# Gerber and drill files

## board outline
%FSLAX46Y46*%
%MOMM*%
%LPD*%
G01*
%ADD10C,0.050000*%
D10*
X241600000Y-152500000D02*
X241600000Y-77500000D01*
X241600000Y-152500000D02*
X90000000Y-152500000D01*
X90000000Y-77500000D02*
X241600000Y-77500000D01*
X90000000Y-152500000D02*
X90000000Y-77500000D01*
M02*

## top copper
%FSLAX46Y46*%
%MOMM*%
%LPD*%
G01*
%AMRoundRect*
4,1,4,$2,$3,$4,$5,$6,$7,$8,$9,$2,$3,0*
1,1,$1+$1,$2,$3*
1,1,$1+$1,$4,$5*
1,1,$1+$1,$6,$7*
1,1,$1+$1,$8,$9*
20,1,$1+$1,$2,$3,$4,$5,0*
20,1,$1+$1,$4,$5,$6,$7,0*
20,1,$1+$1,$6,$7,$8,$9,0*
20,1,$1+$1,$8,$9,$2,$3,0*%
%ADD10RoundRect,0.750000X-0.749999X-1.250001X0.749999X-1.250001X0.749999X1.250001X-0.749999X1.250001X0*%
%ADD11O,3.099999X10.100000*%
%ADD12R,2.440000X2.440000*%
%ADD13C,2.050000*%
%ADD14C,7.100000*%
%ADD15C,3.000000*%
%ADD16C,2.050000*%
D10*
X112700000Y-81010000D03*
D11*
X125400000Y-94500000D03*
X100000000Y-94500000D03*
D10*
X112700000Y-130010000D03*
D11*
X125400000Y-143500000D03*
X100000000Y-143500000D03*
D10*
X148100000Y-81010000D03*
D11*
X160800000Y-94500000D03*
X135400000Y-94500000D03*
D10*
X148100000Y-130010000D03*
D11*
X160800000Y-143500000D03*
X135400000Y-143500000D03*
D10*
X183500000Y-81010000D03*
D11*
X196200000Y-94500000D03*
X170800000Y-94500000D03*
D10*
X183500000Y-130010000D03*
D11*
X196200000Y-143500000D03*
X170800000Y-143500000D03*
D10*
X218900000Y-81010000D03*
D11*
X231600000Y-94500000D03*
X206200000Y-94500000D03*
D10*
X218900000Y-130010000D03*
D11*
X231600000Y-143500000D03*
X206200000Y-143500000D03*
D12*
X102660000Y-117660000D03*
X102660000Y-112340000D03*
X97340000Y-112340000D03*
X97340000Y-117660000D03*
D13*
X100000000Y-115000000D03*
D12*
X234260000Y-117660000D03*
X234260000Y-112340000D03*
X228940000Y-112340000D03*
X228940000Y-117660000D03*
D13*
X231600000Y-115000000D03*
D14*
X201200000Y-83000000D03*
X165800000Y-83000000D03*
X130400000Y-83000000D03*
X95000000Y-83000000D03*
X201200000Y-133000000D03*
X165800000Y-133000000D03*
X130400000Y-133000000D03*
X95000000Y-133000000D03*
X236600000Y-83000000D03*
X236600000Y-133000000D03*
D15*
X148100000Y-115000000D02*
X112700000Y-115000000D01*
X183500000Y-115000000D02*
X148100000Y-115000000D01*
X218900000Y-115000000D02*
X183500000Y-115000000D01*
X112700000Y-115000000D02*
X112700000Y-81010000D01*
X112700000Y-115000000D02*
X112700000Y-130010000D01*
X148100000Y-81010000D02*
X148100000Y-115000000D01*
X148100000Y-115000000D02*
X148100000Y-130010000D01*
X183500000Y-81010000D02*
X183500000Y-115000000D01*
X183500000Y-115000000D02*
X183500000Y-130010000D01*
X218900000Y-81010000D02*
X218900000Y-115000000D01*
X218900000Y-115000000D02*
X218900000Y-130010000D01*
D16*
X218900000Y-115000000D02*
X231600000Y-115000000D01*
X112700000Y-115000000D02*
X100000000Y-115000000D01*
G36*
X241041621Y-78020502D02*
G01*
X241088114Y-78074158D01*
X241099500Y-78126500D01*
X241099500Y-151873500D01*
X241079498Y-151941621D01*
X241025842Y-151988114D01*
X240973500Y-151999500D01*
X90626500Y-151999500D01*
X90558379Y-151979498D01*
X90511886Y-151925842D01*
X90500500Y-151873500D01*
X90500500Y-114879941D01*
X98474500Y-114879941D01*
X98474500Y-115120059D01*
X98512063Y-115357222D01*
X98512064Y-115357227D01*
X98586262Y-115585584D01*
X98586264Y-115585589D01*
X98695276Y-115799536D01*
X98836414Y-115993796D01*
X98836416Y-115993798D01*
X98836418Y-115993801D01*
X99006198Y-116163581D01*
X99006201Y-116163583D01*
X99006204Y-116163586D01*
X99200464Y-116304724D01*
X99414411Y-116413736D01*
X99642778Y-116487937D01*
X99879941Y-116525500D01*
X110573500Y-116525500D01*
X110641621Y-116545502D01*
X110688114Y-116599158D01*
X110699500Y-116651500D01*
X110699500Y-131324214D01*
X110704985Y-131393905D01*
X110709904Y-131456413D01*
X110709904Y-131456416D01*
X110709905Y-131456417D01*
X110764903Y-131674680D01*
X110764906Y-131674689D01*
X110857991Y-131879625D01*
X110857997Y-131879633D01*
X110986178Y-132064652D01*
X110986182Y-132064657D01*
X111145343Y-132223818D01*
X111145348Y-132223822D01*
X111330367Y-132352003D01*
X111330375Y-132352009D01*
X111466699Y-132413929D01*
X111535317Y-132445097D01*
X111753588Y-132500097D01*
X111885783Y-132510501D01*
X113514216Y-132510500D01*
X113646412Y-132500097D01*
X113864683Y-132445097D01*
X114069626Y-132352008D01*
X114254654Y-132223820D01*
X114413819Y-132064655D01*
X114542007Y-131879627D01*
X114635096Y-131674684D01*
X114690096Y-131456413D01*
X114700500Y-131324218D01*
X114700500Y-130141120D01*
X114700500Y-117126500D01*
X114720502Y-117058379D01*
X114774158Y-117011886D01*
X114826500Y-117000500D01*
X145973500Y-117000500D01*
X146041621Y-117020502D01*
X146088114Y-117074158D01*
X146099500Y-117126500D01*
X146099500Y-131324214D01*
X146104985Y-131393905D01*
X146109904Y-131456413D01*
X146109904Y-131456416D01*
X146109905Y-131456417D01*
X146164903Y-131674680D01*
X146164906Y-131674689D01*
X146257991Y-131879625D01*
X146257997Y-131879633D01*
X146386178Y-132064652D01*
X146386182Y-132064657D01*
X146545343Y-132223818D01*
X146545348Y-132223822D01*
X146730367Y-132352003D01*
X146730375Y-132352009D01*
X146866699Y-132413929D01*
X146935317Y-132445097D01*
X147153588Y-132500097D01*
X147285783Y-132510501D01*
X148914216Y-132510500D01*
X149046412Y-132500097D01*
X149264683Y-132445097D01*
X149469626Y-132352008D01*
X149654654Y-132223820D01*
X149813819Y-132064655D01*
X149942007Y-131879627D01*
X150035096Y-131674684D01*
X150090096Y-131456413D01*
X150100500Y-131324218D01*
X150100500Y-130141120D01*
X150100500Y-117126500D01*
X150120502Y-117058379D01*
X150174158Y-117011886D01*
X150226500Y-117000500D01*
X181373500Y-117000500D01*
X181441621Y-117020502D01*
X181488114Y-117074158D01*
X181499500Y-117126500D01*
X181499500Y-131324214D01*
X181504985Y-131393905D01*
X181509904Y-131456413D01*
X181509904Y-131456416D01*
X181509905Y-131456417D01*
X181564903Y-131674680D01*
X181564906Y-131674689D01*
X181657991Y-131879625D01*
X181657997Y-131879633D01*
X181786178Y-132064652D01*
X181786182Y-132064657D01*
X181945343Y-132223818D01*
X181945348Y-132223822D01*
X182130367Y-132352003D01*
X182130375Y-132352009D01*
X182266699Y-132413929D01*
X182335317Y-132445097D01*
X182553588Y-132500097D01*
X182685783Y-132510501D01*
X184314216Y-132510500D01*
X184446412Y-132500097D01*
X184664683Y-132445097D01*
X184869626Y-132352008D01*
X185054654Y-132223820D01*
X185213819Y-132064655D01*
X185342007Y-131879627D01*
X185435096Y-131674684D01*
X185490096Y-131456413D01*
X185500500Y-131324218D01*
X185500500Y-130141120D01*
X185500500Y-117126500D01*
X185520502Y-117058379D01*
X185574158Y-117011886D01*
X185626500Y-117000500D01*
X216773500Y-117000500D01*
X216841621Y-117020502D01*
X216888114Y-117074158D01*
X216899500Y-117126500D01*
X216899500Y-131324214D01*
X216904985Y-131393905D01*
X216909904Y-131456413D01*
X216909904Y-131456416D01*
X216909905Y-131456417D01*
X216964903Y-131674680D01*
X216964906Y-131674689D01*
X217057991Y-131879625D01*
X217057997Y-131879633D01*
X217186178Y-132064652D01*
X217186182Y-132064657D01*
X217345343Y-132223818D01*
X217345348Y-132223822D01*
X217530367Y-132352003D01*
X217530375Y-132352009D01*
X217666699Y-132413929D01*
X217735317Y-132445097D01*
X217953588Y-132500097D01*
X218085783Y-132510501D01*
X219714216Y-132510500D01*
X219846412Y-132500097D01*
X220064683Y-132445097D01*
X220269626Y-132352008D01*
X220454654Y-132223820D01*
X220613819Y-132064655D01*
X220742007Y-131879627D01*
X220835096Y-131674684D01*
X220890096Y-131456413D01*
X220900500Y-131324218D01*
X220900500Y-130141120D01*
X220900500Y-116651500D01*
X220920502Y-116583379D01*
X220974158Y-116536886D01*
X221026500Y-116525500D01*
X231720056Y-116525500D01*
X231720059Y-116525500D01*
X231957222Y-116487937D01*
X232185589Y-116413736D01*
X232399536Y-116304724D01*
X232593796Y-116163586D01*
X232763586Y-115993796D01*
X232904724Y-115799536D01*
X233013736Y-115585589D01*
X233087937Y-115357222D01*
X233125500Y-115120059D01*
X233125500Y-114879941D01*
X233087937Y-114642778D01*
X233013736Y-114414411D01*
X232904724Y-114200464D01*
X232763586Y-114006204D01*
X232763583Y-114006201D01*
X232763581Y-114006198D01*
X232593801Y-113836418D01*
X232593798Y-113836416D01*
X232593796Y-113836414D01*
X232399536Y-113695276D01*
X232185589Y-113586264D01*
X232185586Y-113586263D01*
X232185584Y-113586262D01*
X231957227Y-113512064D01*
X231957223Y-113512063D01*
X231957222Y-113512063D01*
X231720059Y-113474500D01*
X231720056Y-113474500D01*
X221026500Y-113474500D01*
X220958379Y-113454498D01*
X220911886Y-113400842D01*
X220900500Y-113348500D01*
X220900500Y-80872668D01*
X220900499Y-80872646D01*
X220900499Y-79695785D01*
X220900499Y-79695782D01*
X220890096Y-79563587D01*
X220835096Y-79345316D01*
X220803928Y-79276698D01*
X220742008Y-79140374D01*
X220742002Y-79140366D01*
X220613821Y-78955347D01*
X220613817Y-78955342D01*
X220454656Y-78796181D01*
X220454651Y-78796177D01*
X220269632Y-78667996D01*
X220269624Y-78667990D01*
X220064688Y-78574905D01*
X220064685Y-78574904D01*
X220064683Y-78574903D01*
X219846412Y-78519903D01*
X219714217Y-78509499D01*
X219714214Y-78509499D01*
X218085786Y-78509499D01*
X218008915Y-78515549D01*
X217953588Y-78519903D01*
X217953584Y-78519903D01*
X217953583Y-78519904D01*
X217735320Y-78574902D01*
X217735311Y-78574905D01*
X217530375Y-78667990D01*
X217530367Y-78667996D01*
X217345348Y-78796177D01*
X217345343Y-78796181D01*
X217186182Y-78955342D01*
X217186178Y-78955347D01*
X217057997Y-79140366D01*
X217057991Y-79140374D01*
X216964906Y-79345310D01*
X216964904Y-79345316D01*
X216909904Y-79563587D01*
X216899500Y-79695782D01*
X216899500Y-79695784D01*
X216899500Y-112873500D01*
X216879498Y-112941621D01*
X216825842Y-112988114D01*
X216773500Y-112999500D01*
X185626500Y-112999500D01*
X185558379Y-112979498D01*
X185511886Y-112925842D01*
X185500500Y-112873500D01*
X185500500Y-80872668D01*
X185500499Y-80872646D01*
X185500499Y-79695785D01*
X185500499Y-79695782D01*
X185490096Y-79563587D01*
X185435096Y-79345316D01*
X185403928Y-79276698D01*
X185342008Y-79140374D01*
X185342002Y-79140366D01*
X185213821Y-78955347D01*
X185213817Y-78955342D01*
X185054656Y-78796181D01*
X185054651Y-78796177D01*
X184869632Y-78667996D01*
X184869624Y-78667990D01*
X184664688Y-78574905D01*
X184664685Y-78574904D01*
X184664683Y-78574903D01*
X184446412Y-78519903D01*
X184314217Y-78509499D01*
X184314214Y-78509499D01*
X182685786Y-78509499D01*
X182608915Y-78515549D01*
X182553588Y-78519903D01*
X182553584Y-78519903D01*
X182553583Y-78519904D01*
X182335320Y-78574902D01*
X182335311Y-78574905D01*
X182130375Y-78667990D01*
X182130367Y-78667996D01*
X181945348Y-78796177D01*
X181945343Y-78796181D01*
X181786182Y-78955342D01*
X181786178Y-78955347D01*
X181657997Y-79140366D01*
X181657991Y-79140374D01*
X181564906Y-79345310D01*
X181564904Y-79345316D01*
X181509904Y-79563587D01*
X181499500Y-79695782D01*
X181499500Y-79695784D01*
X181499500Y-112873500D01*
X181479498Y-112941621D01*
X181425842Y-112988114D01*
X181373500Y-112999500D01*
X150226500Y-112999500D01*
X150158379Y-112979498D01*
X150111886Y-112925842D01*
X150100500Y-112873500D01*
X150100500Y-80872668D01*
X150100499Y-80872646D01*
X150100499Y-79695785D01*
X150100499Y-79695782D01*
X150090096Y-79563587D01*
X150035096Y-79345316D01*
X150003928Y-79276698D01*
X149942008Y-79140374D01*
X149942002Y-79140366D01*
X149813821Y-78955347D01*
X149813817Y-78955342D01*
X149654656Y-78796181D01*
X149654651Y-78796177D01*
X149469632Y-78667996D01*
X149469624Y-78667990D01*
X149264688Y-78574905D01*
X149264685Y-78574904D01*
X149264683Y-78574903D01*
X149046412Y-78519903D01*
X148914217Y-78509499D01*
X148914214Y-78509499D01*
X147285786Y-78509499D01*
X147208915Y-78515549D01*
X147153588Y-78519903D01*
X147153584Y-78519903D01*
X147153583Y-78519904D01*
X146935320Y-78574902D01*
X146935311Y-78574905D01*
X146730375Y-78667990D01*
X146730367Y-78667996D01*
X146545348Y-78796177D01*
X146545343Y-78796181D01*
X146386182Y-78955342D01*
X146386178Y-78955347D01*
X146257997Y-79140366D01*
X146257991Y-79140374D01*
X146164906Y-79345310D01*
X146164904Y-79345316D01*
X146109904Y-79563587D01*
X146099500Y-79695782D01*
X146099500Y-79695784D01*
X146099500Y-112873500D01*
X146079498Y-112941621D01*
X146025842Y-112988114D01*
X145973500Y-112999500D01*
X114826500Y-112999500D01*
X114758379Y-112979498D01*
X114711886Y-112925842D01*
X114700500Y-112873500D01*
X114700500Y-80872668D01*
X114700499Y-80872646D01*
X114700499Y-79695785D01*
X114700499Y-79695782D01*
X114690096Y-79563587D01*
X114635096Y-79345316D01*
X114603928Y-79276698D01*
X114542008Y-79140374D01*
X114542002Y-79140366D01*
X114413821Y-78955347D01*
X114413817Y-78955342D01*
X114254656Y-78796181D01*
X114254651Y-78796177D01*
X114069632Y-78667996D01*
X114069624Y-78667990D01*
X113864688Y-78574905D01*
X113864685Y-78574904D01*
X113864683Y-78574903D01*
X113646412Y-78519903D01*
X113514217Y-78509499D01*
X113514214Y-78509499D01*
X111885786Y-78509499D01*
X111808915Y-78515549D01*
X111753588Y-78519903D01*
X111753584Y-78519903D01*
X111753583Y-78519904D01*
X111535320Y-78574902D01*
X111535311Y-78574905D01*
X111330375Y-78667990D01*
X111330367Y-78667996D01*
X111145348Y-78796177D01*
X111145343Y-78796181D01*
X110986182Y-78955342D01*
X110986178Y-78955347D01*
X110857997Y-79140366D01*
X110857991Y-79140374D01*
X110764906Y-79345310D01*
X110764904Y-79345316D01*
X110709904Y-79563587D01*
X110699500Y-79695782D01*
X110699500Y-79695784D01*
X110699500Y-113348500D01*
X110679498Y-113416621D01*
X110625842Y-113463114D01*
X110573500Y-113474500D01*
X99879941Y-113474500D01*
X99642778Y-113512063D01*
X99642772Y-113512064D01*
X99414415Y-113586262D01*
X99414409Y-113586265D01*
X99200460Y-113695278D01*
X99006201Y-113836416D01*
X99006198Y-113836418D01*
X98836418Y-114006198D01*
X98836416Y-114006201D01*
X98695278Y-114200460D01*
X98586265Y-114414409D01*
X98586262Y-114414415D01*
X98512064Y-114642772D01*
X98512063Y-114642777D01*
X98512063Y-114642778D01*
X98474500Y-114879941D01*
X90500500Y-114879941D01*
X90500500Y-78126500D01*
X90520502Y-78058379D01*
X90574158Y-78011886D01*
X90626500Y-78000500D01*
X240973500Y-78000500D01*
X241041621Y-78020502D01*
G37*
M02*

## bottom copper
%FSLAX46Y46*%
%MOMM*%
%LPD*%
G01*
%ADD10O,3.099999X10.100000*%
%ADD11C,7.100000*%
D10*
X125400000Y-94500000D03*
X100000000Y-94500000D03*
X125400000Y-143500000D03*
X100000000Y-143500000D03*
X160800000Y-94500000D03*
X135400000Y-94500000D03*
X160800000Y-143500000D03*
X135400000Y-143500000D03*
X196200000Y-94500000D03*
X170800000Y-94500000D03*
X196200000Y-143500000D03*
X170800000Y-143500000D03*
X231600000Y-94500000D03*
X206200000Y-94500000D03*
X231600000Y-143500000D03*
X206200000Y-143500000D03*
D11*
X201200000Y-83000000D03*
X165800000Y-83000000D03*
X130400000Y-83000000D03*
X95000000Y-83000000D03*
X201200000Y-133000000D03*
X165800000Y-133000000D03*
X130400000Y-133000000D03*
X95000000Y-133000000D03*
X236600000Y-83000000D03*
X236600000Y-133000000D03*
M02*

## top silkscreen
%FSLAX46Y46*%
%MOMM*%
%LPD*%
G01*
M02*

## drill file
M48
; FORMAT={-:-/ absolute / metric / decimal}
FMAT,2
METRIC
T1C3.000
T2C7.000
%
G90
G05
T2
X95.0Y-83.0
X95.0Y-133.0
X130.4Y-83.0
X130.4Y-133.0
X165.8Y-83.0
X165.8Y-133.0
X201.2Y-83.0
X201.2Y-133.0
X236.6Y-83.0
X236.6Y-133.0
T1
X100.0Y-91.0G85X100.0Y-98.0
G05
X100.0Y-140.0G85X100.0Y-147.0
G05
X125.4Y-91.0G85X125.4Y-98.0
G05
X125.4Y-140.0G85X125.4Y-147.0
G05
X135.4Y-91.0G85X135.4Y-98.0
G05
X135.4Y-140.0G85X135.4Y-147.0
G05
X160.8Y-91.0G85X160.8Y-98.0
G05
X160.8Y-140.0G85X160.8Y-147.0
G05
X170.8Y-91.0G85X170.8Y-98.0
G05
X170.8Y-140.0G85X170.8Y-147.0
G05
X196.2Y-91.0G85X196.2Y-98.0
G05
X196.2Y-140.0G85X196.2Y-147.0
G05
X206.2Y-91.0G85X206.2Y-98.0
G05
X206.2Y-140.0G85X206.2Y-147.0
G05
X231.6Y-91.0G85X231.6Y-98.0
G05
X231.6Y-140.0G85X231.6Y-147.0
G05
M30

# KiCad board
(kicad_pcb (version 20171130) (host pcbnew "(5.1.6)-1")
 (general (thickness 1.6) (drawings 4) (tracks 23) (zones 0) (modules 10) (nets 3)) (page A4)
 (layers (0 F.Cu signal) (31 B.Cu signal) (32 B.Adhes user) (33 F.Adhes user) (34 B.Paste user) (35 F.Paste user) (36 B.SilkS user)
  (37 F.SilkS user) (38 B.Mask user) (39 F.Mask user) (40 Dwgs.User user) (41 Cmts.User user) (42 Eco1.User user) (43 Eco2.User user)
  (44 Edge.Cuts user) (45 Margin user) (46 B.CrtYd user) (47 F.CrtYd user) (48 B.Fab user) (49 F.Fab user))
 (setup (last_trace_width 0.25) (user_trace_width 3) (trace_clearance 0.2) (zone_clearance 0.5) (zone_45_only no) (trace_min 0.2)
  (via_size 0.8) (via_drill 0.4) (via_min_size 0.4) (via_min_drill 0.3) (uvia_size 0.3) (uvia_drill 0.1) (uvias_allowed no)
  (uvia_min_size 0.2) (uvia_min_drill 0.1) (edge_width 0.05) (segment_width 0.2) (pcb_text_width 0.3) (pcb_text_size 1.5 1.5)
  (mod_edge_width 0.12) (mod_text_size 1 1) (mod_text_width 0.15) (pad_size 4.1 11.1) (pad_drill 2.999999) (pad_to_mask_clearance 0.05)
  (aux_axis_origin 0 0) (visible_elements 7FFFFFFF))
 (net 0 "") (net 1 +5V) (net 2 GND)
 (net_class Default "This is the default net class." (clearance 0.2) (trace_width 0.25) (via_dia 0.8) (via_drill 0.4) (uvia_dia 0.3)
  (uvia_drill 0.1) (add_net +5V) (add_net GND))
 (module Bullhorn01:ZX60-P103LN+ (layer F.Cu) (at 112.7 94.5)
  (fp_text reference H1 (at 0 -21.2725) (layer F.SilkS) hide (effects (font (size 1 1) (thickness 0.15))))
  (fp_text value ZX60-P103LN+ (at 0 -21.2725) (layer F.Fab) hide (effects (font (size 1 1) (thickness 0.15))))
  (pad 2 smd roundrect (at 0 -13.49) (size 2.999999 4.000002) (layers F.Cu F.Paste F.Mask) (roundrect_rratio 0.25) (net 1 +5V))
  (pad 1 thru_hole oval (at 12.7 0) (size 3.099999 10.1) (drill oval 2.999999 10) (layers *.Cu *.Mask) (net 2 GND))
  (pad 1 thru_hole oval (at -12.7 0) (size 3.099999 10.1) (drill oval 2.999999 10) (layers *.Cu *.Mask) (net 2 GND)))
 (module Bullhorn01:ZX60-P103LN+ (layer F.Cu) (at 112.7 143.5)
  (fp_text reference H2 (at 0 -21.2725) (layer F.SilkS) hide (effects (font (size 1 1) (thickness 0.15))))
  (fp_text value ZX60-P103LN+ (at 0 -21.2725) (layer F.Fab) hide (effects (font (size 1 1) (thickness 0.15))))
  (pad 2 smd roundrect (at 0 -13.49) (size 2.999999 4.000002) (layers F.Cu F.Paste F.Mask) (roundrect_rratio 0.25) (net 1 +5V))
  (pad 1 thru_hole oval (at 12.7 0) (size 3.099999 10.1) (drill oval 2.999999 10) (layers *.Cu *.Mask) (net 2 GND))
  (pad 1 thru_hole oval (at -12.7 0) (size 3.099999 10.1) (drill oval 2.999999 10) (layers *.Cu *.Mask) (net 2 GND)))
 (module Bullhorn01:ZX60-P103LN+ (layer F.Cu) (at 148.1 94.5)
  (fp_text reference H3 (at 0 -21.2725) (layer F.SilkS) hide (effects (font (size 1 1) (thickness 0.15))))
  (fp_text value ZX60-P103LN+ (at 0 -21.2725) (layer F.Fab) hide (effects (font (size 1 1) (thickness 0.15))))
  (pad 2 smd roundrect (at 0 -13.49) (size 2.999999 4.000002) (layers F.Cu F.Paste F.Mask) (roundrect_rratio 0.25) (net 1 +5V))
  (pad 1 thru_hole oval (at 12.7 0) (size 3.099999 10.1) (drill oval 2.999999 10) (layers *.Cu *.Mask) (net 2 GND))
  (pad 1 thru_hole oval (at -12.7 0) (size 3.099999 10.1) (drill oval 2.999999 10) (layers *.Cu *.Mask) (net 2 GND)))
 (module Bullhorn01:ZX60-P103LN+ (layer F.Cu) (at 148.1 143.5)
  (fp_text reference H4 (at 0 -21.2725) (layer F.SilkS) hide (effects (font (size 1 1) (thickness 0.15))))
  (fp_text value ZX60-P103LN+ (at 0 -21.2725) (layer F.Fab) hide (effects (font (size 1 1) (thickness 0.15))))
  (pad 2 smd roundrect (at 0 -13.49) (size 2.999999 4.000002) (layers F.Cu F.Paste F.Mask) (roundrect_rratio 0.25) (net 1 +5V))
  (pad 1 thru_hole oval (at 12.7 0) (size 3.099999 10.1) (drill oval 2.999999 10) (layers *.Cu *.Mask) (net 2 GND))
  (pad 1 thru_hole oval (at -12.7 0) (size 3.099999 10.1) (drill oval 2.999999 10) (layers *.Cu *.Mask) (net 2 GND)))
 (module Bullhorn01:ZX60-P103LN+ (layer F.Cu) (at 183.5 94.5)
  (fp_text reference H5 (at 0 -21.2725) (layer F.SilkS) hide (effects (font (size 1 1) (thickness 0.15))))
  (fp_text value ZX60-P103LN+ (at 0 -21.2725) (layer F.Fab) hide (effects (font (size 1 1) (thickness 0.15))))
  (pad 2 smd roundrect (at 0 -13.49) (size 2.999999 4.000002) (layers F.Cu F.Paste F.Mask) (roundrect_rratio 0.25) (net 1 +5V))
  (pad 1 thru_hole oval (at 12.7 0) (size 3.099999 10.1) (drill oval 2.999999 10) (layers *.Cu *.Mask) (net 2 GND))
  (pad 1 thru_hole oval (at -12.7 0) (size 3.099999 10.1) (drill oval 2.999999 10) (layers *.Cu *.Mask) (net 2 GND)))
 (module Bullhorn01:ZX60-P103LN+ (layer F.Cu) (at 183.5 143.5)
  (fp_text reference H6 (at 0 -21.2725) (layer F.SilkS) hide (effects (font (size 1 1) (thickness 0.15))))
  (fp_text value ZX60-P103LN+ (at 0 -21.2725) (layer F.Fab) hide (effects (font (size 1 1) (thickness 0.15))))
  (pad 2 smd roundrect (at 0 -13.49) (size 2.999999 4.000002) (layers F.Cu F.Paste F.Mask) (roundrect_rratio 0.25) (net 1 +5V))
  (pad 1 thru_hole oval (at 12.7 0) (size 3.099999 10.1) (drill oval 2.999999 10) (layers *.Cu *.Mask) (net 2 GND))
  (pad 1 thru_hole oval (at -12.7 0) (size 3.099999 10.1) (drill oval 2.999999 10) (layers *.Cu *.Mask) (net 2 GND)))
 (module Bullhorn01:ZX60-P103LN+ (layer F.Cu) (at 218.9 94.5)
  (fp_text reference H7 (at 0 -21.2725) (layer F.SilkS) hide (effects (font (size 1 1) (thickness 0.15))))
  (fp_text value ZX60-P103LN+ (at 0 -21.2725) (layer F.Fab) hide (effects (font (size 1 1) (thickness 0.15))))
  (pad 2 smd roundrect (at 0 -13.49) (size 2.999999 4.000002) (layers F.Cu F.Paste F.Mask) (roundrect_rratio 0.25) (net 1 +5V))
  (pad 1 thru_hole oval (at 12.7 0) (size 3.099999 10.1) (drill oval 2.999999 10) (layers *.Cu *.Mask) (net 2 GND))
  (pad 1 thru_hole oval (at -12.7 0) (size 3.099999 10.1) (drill oval 2.999999 10) (layers *.Cu *.Mask) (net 2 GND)))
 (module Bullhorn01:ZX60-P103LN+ (layer F.Cu) (at 218.9 143.5)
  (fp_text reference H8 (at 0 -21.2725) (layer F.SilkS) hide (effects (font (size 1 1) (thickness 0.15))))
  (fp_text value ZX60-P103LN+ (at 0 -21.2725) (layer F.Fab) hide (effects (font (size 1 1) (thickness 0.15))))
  (pad 2 smd roundrect (at 0 -13.49) (size 2.999999 4.000002) (layers F.Cu F.Paste F.Mask) (roundrect_rratio 0.25) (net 1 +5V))
  (pad 1 thru_hole oval (at 12.7 0) (size 3.099999 10.1) (drill oval 2.999999 10) (layers *.Cu *.Mask) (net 2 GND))
  (pad 1 thru_hole oval (at -12.7 0) (size 3.099999 10.1) (drill oval 2.999999 10) (layers *.Cu *.Mask) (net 2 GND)))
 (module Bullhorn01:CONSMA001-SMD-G (layer F.Cu) (at 100 115)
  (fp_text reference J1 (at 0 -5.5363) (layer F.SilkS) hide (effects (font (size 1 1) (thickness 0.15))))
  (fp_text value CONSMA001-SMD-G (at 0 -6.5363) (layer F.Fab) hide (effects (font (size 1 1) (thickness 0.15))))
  (pad 2 smd rect (at 2.66 2.66) (size 2.44 2.44) (layers F.Cu F.Paste F.Mask) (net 2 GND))
  (pad 2 smd rect (at 2.66 -2.66) (size 2.44 2.44) (layers F.Cu F.Paste F.Mask) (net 2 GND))
  (pad 2 smd rect (at -2.66 -2.66 90) (size 2.44 2.44) (layers F.Cu F.Paste F.Mask) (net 2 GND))
  (pad 2 smd rect (at -2.66 2.66) (size 2.44 2.44) (layers F.Cu F.Paste F.Mask) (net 2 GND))
  (pad 1 smd circle (at 0 0) (size 2.05 2.05) (layers F.Cu F.Paste F.Mask) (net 1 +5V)))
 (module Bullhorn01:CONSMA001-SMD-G (layer F.Cu) (at 231.6 115)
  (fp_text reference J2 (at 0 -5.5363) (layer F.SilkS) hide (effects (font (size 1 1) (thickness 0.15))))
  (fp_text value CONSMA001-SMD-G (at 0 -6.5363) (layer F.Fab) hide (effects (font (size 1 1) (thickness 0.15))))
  (pad 2 smd rect (at 2.66 2.66) (size 2.44 2.44) (layers F.Cu F.Paste F.Mask) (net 2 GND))
  (pad 2 smd rect (at 2.66 -2.66) (size 2.44 2.44) (layers F.Cu F.Paste F.Mask) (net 2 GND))
  (pad 2 smd rect (at -2.66 -2.66 90) (size 2.44 2.44) (layers F.Cu F.Paste F.Mask) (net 2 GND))
  (pad 2 smd rect (at -2.66 2.66) (size 2.44 2.44) (layers F.Cu F.Paste F.Mask) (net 2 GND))
  (pad 1 smd circle (at 0 0) (size 2.05 2.05) (layers F.Cu F.Paste F.Mask) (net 1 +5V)))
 (gr_line (start 241.6 152.5) (end 241.6 77.5) (layer Edge.Cuts) (width 0.05))
 (gr_line (start 241.6 152.5) (end 90 152.5) (layer Edge.Cuts) (width 0.05))
 (gr_line (start 90 77.5) (end 241.6 77.5) (layer Edge.Cuts) (width 0.05))
 (gr_line (start 90 152.5) (end 90 77.5) (layer Edge.Cuts) (width 0.05))
 (via (at 201.2 83) (size 7.1) (drill 7) (layers F.Cu B.Cu) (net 2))
 (via (at 165.8 83) (size 7.1) (drill 7) (layers F.Cu B.Cu) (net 2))
 (via (at 130.4 83) (size 7.1) (drill 7) (layers F.Cu B.Cu) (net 2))
 (via (at 95 83) (size 7.1) (drill 7) (layers F.Cu B.Cu) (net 2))
 (via (at 201.2 133) (size 7.1) (drill 7) (layers F.Cu B.Cu) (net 2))
 (via (at 165.8 133) (size 7.1) (drill 7) (layers F.Cu B.Cu) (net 2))
 (via (at 130.4 133) (size 7.1) (drill 7) (layers F.Cu B.Cu) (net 2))
 (via (at 95 133) (size 7.1) (drill 7) (layers F.Cu B.Cu) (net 2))
 (via (at 236.6 83) (size 7.1) (drill 7) (layers F.Cu B.Cu) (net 2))
 (via (at 236.6 133) (size 7.1) (drill 7) (layers F.Cu B.Cu) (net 2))
 (segment (start 148.1 115) (end 112.7 115) (width 3) (layer F.Cu) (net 1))
 (segment (start 183.5 115) (end 148.1 115) (width 3) (layer F.Cu) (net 1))
 (segment (start 218.9 115) (end 183.5 115) (width 3) (layer F.Cu) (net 1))
 (segment (start 112.7 115) (end 112.7 81.01) (width 3) (layer F.Cu) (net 1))
 (segment (start 112.7 115) (end 112.7 130.01) (width 3) (layer F.Cu) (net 1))
 (segment (start 148.1 81.01) (end 148.1 115) (width 3) (layer F.Cu) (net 1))
 (segment (start 148.1 115) (end 148.1 130.01) (width 3) (layer F.Cu) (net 1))
 (segment (start 183.5 81.01) (end 183.5 115) (width 3) (layer F.Cu) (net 1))
 (segment (start 183.5 115) (end 183.5 130.01) (width 3) (layer F.Cu) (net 1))
 (segment (start 218.9 81.01) (end 218.9 115) (width 3) (layer F.Cu) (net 1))
 (segment (start 218.9 115) (end 218.9 130.01) (width 3) (layer F.Cu) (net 1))
 (segment (start 218.9 115) (end 231.6 115) (width 2.05) (layer F.Cu) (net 1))
 (segment (start 112.7 115) (end 100 115) (width 2.05) (layer F.Cu) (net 1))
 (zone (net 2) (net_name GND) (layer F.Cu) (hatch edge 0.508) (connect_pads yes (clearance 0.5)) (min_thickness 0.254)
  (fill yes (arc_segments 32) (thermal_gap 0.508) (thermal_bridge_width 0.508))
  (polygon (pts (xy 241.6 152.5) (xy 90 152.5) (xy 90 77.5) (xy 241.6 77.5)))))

